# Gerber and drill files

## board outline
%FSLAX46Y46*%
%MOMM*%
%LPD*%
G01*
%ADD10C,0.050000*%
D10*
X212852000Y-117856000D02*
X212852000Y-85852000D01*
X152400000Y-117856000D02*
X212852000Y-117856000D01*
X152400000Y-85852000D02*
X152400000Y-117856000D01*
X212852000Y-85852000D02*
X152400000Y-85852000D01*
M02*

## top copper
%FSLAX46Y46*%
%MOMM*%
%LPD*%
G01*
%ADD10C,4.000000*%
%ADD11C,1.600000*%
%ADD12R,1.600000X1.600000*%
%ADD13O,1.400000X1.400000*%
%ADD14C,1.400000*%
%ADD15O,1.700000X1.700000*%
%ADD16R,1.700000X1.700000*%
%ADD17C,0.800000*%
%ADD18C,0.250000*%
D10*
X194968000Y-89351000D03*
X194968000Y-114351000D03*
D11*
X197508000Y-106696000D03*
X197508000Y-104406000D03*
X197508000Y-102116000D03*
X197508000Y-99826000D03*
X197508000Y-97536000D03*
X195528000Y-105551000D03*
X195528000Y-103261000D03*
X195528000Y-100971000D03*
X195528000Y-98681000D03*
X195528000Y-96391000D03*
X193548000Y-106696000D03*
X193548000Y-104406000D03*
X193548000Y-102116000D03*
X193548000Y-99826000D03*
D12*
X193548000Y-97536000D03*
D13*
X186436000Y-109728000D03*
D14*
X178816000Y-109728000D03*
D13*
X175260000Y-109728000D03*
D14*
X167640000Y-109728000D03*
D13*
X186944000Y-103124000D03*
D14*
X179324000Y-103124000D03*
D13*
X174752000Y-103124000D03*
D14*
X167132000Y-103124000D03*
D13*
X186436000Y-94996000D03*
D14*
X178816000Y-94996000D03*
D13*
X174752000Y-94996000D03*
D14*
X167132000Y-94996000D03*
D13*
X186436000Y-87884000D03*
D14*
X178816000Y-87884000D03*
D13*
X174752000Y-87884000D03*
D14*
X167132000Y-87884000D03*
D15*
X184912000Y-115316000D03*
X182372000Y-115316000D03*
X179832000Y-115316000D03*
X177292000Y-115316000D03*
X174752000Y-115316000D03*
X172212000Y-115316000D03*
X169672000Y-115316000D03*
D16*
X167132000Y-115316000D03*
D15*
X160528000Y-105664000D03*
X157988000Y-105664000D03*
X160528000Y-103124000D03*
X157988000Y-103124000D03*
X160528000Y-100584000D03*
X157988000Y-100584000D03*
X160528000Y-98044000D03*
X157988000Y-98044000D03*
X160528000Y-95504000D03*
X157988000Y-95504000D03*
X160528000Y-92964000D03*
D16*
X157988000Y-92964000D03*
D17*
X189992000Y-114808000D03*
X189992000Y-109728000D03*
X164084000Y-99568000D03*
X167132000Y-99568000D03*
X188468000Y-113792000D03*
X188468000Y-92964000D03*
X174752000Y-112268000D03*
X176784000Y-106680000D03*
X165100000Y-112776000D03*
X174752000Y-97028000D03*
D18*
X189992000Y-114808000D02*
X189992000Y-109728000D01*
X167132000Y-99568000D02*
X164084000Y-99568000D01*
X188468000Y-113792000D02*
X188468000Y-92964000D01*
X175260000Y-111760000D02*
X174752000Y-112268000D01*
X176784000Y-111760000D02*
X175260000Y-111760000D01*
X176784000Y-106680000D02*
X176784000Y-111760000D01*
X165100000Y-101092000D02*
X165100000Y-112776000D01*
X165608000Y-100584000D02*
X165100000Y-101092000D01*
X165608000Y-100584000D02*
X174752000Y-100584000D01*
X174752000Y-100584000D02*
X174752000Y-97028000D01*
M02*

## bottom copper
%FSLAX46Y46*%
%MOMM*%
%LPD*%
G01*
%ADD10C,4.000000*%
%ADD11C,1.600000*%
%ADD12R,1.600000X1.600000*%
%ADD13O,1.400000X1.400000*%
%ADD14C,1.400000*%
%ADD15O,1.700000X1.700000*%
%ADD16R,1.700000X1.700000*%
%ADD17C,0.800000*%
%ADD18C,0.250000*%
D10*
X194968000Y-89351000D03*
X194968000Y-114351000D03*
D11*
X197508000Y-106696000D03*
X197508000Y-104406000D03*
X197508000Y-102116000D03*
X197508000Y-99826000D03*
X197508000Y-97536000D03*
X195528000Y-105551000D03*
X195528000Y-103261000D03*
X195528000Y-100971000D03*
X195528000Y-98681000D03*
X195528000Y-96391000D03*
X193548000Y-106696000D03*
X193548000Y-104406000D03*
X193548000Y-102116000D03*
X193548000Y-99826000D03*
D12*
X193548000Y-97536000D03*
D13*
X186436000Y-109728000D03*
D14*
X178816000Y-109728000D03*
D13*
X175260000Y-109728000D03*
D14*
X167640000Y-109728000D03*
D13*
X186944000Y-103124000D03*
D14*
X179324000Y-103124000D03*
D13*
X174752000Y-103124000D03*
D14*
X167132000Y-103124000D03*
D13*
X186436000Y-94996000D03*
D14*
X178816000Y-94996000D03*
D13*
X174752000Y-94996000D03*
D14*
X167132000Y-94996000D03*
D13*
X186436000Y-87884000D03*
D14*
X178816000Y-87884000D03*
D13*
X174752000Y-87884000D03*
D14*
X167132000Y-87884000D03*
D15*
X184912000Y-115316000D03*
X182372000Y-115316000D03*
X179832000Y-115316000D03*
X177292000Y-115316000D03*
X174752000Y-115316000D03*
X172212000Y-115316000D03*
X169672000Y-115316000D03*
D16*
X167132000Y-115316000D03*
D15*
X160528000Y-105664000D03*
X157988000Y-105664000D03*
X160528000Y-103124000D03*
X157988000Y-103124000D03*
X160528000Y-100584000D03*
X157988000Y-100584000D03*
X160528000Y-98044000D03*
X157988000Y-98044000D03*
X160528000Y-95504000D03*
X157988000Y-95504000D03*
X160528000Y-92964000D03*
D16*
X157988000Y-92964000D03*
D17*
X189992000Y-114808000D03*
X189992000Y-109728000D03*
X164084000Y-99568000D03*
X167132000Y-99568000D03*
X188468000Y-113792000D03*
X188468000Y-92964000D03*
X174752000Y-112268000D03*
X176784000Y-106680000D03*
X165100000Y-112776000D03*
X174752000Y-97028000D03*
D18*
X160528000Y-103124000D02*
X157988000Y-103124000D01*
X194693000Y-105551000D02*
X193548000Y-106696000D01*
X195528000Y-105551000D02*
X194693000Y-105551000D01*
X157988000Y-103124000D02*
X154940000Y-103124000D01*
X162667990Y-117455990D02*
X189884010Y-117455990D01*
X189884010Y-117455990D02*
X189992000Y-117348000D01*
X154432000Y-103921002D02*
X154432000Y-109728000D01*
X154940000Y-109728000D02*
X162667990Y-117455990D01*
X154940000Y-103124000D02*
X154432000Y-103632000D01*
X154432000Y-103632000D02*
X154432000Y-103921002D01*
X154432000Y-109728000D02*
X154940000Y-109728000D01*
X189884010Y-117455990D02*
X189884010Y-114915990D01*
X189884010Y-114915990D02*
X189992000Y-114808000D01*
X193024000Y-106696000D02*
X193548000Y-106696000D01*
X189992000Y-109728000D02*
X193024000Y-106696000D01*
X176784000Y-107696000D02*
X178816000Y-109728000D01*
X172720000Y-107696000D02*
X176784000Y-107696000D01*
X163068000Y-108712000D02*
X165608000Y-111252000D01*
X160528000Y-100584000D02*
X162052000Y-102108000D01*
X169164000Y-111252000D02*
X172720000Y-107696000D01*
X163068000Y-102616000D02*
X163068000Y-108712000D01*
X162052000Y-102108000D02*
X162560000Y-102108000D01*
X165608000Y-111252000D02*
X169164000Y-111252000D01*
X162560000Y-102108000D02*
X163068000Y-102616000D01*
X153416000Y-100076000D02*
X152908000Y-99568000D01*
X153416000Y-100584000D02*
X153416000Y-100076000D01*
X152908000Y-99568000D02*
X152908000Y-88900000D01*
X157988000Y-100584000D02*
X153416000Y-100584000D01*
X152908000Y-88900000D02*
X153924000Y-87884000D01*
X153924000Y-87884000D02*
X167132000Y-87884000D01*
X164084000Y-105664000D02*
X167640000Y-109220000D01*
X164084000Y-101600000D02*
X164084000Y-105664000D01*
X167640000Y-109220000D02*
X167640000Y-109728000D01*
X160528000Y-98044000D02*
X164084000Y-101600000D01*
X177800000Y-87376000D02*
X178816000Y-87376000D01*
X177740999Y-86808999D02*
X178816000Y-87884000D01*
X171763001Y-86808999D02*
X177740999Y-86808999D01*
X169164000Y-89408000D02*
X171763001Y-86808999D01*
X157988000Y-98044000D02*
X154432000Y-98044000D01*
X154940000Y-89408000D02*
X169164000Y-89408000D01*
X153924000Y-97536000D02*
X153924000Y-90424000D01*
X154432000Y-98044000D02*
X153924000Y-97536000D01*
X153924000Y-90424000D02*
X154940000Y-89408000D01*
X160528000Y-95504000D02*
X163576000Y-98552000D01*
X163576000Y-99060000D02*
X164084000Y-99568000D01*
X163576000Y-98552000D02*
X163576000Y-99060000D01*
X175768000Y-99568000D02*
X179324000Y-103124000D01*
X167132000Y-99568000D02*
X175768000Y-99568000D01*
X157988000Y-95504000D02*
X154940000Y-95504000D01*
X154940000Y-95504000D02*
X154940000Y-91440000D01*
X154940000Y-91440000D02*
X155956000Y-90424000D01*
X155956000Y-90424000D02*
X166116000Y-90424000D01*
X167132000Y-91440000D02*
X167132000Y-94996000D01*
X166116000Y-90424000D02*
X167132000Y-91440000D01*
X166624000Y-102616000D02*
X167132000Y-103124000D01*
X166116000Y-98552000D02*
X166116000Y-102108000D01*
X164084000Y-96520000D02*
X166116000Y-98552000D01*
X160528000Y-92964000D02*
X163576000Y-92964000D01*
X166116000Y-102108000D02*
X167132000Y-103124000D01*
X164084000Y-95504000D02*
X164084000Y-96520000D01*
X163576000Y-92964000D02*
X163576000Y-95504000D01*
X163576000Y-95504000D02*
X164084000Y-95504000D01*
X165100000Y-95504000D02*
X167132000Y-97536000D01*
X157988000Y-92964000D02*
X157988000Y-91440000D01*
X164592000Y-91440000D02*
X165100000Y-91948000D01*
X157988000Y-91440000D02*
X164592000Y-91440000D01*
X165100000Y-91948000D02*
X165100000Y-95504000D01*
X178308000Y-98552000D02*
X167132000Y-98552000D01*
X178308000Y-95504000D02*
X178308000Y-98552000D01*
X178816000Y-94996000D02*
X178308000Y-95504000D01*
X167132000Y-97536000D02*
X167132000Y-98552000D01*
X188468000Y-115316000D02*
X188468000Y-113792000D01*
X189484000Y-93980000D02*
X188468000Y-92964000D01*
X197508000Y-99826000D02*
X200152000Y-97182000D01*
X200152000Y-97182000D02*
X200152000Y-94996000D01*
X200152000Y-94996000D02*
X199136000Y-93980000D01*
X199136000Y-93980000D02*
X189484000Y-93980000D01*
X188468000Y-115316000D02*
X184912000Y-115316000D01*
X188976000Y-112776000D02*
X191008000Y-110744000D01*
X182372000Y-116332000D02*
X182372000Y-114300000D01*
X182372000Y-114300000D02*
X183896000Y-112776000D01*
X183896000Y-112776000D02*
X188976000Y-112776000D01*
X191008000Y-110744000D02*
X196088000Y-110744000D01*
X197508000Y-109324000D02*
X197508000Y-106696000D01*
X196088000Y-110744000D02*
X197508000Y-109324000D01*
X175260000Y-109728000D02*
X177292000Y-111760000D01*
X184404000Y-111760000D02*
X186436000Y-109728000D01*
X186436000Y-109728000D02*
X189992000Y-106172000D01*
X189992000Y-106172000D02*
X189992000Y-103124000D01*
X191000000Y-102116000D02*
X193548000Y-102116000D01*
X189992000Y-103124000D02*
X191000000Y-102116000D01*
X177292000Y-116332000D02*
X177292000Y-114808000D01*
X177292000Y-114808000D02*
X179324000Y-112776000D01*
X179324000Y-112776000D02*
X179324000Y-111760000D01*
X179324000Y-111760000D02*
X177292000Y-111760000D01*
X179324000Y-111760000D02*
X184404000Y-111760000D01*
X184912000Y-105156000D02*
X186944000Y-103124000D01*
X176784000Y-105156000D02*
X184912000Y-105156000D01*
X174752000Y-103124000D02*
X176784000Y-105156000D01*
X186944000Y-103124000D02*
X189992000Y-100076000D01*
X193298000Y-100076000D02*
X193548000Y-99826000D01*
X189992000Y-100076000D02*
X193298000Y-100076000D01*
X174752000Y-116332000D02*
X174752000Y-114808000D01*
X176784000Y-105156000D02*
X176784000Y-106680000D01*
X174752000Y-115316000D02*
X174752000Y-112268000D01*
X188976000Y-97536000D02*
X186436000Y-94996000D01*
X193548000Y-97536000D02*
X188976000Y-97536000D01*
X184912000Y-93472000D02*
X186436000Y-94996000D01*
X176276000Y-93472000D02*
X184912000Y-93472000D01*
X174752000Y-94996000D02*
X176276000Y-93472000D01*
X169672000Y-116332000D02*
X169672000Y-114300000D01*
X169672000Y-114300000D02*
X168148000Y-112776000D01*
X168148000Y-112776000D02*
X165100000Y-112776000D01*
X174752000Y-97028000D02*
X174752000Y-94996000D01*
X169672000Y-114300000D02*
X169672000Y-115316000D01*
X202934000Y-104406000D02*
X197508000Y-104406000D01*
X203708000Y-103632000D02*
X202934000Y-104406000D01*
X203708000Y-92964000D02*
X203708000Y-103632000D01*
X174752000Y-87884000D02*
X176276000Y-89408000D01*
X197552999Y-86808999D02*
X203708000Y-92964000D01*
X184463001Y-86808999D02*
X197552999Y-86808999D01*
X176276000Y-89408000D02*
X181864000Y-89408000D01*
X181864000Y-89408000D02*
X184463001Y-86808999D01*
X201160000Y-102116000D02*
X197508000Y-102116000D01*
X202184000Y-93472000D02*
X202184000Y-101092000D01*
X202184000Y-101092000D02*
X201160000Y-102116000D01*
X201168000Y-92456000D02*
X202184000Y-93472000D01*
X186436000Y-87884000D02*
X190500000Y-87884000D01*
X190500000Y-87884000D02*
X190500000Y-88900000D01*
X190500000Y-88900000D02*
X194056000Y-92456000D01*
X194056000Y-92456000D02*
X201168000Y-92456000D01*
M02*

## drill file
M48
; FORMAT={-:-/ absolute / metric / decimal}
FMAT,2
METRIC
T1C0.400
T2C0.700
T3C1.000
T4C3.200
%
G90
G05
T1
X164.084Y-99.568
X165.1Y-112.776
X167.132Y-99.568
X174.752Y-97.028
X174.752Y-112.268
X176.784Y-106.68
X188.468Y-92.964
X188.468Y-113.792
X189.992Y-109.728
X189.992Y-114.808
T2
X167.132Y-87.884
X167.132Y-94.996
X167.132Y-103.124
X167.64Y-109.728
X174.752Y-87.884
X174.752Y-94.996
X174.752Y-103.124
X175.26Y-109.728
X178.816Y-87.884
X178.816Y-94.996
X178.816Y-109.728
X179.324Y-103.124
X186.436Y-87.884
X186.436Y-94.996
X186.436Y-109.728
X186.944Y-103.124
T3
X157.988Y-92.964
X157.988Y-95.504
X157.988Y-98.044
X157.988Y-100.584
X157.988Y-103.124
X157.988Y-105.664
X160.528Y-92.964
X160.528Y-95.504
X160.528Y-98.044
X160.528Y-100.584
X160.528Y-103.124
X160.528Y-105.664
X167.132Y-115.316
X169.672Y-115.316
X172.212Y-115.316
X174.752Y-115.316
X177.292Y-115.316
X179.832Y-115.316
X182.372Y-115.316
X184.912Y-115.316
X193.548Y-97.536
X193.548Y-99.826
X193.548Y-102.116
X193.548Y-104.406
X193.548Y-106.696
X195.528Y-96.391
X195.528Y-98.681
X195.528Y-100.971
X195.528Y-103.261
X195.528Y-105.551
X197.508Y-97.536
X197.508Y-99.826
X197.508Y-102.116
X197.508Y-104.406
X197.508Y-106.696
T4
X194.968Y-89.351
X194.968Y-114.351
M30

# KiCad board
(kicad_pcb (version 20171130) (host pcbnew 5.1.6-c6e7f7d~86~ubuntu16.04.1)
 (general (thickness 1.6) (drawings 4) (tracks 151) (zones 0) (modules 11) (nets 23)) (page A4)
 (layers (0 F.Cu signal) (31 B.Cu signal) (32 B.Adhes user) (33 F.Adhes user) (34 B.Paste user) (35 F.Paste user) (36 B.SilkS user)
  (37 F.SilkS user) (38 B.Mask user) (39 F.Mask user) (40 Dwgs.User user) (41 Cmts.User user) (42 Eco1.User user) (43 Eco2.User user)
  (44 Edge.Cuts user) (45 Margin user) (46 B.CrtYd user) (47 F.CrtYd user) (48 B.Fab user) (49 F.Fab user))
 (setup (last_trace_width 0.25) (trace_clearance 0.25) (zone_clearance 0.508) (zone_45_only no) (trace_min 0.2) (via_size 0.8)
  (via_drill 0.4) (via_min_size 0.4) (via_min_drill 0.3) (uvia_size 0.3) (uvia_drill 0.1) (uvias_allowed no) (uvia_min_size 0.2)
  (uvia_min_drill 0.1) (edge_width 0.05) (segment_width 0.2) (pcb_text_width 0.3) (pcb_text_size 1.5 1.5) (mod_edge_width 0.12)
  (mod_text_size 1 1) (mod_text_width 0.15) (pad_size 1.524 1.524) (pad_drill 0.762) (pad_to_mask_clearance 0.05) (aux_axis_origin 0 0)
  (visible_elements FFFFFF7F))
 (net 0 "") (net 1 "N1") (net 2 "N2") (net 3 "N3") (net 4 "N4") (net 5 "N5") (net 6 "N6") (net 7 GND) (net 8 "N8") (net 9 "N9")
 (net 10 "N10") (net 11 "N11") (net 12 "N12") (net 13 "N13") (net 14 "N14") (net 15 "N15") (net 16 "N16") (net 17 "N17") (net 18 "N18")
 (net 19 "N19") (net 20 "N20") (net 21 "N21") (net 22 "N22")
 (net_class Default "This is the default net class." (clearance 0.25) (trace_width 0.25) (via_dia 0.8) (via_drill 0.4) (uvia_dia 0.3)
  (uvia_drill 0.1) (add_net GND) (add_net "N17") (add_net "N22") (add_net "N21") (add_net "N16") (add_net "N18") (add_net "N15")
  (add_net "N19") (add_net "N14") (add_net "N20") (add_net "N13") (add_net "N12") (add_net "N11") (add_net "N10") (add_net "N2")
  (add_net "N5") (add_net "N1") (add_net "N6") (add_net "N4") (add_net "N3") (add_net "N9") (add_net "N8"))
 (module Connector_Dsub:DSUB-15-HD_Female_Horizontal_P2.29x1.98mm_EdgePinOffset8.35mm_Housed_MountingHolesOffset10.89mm (layer F.Cu)
  (at 193.548 97.536 90)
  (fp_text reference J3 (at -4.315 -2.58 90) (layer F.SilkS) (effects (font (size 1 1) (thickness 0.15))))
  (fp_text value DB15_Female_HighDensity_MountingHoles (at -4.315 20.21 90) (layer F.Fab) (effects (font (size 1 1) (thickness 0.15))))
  (pad 0 thru_hole circle (at 8.185 1.42 90) (size 4 4) (drill 3.2) (layers *.Cu *.Mask) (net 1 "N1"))
  (pad 0 thru_hole circle (at -16.815 1.42 90) (size 4 4) (drill 3.2) (layers *.Cu *.Mask) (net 1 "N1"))
  (pad 15 thru_hole circle (at -9.16 3.96 90) (size 1.6 1.6) (drill 1) (layers *.Cu *.Mask) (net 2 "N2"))
  (pad 14 thru_hole circle (at -6.87 3.96 90) (size 1.6 1.6) (drill 1) (layers *.Cu *.Mask) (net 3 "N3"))
  (pad 13 thru_hole circle (at -4.58 3.96 90) (size 1.6 1.6) (drill 1) (layers *.Cu *.Mask) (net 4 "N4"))
  (pad 12 thru_hole circle (at -2.29 3.96 90) (size 1.6 1.6) (drill 1) (layers *.Cu *.Mask) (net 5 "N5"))
  (pad 11 thru_hole circle (at 0 3.96 90) (size 1.6 1.6) (drill 1) (layers *.Cu *.Mask) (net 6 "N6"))
  (pad 10 thru_hole circle (at -8.015 1.98 90) (size 1.6 1.6) (drill 1) (layers *.Cu *.Mask) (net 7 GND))
  (pad 9 thru_hole circle (at -5.725 1.98 90) (size 1.6 1.6) (drill 1) (layers *.Cu *.Mask) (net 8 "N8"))
  (pad 8 thru_hole circle (at -3.435 1.98 90) (size 1.6 1.6) (drill 1) (layers *.Cu *.Mask) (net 7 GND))
  (pad 7 thru_hole circle (at -1.145 1.98 90) (size 1.6 1.6) (drill 1) (layers *.Cu *.Mask) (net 7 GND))
  (pad 6 thru_hole circle (at 1.145 1.98 90) (size 1.6 1.6) (drill 1) (layers *.Cu *.Mask) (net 7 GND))
  (pad 5 thru_hole circle (at -9.16 0 90) (size 1.6 1.6) (drill 1) (layers *.Cu *.Mask) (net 7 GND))
  (pad 4 thru_hole circle (at -6.87 0 90) (size 1.6 1.6) (drill 1) (layers *.Cu *.Mask) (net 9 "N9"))
  (pad 3 thru_hole circle (at -4.58 0 90) (size 1.6 1.6) (drill 1) (layers *.Cu *.Mask) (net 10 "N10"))
  (pad 2 thru_hole circle (at -2.29 0 90) (size 1.6 1.6) (drill 1) (layers *.Cu *.Mask) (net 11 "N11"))
  (pad 1 thru_hole rect (at 0 0 90) (size 1.6 1.6) (drill 1) (layers *.Cu *.Mask) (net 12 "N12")))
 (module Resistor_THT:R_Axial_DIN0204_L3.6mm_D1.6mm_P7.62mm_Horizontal (layer F.Cu) (at 178.816 109.728)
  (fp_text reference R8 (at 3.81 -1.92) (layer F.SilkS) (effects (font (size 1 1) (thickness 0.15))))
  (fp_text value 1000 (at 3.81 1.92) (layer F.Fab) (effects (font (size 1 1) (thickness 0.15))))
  (pad 2 thru_hole oval (at 7.62 0) (size 1.4 1.4) (drill 0.7) (layers *.Cu *.Mask) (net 10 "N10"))
  (pad 1 thru_hole circle (at 0 0) (size 1.4 1.4) (drill 0.7) (layers *.Cu *.Mask) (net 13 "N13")))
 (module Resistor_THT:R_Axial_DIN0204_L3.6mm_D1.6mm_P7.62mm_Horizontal (layer F.Cu) (at 167.64 109.728)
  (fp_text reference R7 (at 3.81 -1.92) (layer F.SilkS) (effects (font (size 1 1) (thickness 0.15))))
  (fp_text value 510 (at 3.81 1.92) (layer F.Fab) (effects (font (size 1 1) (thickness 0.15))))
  (pad 2 thru_hole oval (at 7.62 0) (size 1.4 1.4) (drill 0.7) (layers *.Cu *.Mask) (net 10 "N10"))
  (pad 1 thru_hole circle (at 0 0) (size 1.4 1.4) (drill 0.7) (layers *.Cu *.Mask) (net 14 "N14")))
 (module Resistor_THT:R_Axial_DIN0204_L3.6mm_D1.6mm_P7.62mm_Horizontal (layer F.Cu) (at 179.324 103.124)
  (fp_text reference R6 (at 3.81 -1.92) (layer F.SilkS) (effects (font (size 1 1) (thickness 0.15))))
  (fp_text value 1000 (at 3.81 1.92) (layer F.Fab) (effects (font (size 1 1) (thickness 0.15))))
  (pad 2 thru_hole oval (at 7.62 0) (size 1.4 1.4) (drill 0.7) (layers *.Cu *.Mask) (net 11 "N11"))
  (pad 1 thru_hole circle (at 0 0) (size 1.4 1.4) (drill 0.7) (layers *.Cu *.Mask) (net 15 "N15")))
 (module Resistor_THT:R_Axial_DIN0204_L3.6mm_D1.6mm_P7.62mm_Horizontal (layer F.Cu) (at 167.132 103.124)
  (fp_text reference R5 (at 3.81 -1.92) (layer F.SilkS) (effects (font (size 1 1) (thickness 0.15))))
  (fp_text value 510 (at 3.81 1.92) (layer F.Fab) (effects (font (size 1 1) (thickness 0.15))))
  (pad 2 thru_hole oval (at 7.62 0) (size 1.4 1.4) (drill 0.7) (layers *.Cu *.Mask) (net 11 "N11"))
  (pad 1 thru_hole circle (at 0 0) (size 1.4 1.4) (drill 0.7) (layers *.Cu *.Mask) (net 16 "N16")))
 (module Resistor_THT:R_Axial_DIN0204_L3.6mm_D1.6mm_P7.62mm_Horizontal (layer F.Cu) (at 178.816 94.996)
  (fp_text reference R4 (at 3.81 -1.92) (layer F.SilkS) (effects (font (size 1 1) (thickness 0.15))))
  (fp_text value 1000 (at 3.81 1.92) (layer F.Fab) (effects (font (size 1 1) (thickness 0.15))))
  (pad 2 thru_hole oval (at 7.62 0) (size 1.4 1.4) (drill 0.7) (layers *.Cu *.Mask) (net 12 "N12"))
  (pad 1 thru_hole circle (at 0 0) (size 1.4 1.4) (drill 0.7) (layers *.Cu *.Mask) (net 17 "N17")))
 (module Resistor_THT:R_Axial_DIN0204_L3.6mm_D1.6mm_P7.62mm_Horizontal (layer F.Cu) (at 167.132 94.996)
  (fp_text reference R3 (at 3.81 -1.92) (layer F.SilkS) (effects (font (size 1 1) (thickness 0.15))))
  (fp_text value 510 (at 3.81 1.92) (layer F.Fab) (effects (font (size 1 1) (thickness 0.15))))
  (pad 2 thru_hole oval (at 7.62 0) (size 1.4 1.4) (drill 0.7) (layers *.Cu *.Mask) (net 12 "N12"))
  (pad 1 thru_hole circle (at 0 0) (size 1.4 1.4) (drill 0.7) (layers *.Cu *.Mask) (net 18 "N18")))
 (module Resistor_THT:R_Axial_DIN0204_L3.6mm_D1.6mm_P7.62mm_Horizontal (layer F.Cu) (at 178.816 87.884)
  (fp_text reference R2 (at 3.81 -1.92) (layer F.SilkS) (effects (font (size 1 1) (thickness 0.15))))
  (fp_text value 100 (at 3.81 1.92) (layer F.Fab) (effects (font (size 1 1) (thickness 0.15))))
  (pad 2 thru_hole oval (at 7.62 0) (size 1.4 1.4) (drill 0.7) (layers *.Cu *.Mask) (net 4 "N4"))
  (pad 1 thru_hole circle (at 0 0) (size 1.4 1.4) (drill 0.7) (layers *.Cu *.Mask) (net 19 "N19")))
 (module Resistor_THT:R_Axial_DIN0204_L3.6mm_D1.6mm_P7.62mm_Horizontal (layer F.Cu) (at 167.132 87.884)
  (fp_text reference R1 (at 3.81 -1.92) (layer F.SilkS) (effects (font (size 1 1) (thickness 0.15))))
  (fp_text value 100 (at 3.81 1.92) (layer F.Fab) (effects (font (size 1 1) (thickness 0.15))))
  (pad 2 thru_hole oval (at 7.62 0) (size 1.4 1.4) (drill 0.7) (layers *.Cu *.Mask) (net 3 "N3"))
  (pad 1 thru_hole circle (at 0 0) (size 1.4 1.4) (drill 0.7) (layers *.Cu *.Mask) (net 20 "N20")))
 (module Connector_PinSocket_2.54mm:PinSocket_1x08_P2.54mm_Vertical (layer F.Cu) (at 167.132 115.316 90)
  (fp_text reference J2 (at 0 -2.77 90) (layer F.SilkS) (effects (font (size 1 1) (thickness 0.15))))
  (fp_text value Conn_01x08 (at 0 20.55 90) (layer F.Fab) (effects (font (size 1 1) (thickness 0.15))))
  (pad 8 thru_hole oval (at 0 17.78 90) (size 1.7 1.7) (drill 1) (layers *.Cu *.Mask) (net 5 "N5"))
  (pad 7 thru_hole oval (at 0 15.24 90) (size 1.7 1.7) (drill 1) (layers *.Cu *.Mask) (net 2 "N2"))
  (pad 6 thru_hole oval (at 0 12.7 90) (size 1.7 1.7) (drill 1) (layers *.Cu *.Mask) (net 10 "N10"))
  (pad 5 thru_hole oval (at 0 10.16 90) (size 1.7 1.7) (drill 1) (layers *.Cu *.Mask) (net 10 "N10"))
  (pad 4 thru_hole oval (at 0 7.62 90) (size 1.7 1.7) (drill 1) (layers *.Cu *.Mask) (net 11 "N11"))
  (pad 3 thru_hole oval (at 0 5.08 90) (size 1.7 1.7) (drill 1) (layers *.Cu *.Mask) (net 11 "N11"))
  (pad 2 thru_hole oval (at 0 2.54 90) (size 1.7 1.7) (drill 1) (layers *.Cu *.Mask) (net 12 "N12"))
  (pad 1 thru_hole rect (at 0 0 90) (size 1.7 1.7) (drill 1) (layers *.Cu *.Mask) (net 12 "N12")))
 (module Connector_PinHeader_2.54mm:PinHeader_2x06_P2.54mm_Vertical (layer F.Cu) (at 157.988 92.964)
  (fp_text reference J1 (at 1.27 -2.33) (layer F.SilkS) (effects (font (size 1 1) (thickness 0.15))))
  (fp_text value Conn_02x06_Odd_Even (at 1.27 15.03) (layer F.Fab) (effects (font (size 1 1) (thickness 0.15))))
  (pad 12 thru_hole oval (at 2.54 12.7) (size 1.7 1.7) (drill 1) (layers *.Cu *.Mask) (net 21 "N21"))
  (pad 11 thru_hole oval (at 0 12.7) (size 1.7 1.7) (drill 1) (layers *.Cu *.Mask) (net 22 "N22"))
  (pad 10 thru_hole oval (at 2.54 10.16) (size 1.7 1.7) (drill 1) (layers *.Cu *.Mask) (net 7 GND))
  (pad 9 thru_hole oval (at 0 10.16) (size 1.7 1.7) (drill 1) (layers *.Cu *.Mask) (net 7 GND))
  (pad 8 thru_hole oval (at 2.54 7.62) (size 1.7 1.7) (drill 1) (layers *.Cu *.Mask) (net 13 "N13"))
  (pad 7 thru_hole oval (at 0 7.62) (size 1.7 1.7) (drill 1) (layers *.Cu *.Mask) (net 20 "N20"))
  (pad 6 thru_hole oval (at 2.54 5.08) (size 1.7 1.7) (drill 1) (layers *.Cu *.Mask) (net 14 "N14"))
  (pad 5 thru_hole oval (at 0 5.08) (size 1.7 1.7) (drill 1) (layers *.Cu *.Mask) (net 19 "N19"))
  (pad 4 thru_hole oval (at 2.54 2.54) (size 1.7 1.7) (drill 1) (layers *.Cu *.Mask) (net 15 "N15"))
  (pad 3 thru_hole oval (at 0 2.54) (size 1.7 1.7) (drill 1) (layers *.Cu *.Mask) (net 18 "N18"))
  (pad 2 thru_hole oval (at 2.54 0) (size 1.7 1.7) (drill 1) (layers *.Cu *.Mask) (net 16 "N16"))
  (pad 1 thru_hole rect (at 0 0) (size 1.7 1.7) (drill 1) (layers *.Cu *.Mask) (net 17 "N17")))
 (gr_line (start 212.852 117.856) (end 212.852 85.852) (layer Edge.Cuts) (width 0.05))
 (gr_line (start 152.4 117.856) (end 212.852 117.856) (layer Edge.Cuts) (width 0.05))
 (gr_line (start 152.4 85.852) (end 152.4 117.856) (layer Edge.Cuts) (width 0.05))
 (gr_line (start 212.852 85.852) (end 152.4 85.852) (layer Edge.Cuts) (width 0.05))
 (segment (start 160.528 103.124) (end 157.988 103.124) (width 0.25) (layer B.Cu) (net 7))
 (segment (start 194.693 105.551) (end 193.548 106.696) (width 0.25) (layer B.Cu) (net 7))
 (segment (start 195.528 105.551) (end 194.693 105.551) (width 0.25) (layer B.Cu) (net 7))
 (segment (start 157.988 103.124) (end 154.94 103.124) (width 0.25) (layer B.Cu) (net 7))
 (segment (start 162.66799 117.45599) (end 189.88401 117.45599) (width 0.25) (layer B.Cu) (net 7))
 (segment (start 189.88401 117.45599) (end 189.992 117.348) (width 0.25) (layer B.Cu) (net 7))
 (segment (start 154.432 103.921002) (end 154.432 109.728) (width 0.25) (layer B.Cu) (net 7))
 (segment (start 154.94 109.728) (end 162.66799 117.45599) (width 0.25) (layer B.Cu) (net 7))
 (segment (start 154.94 103.124) (end 154.432 103.632) (width 0.25) (layer B.Cu) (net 7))
 (segment (start 154.432 103.632) (end 154.432 103.921002) (width 0.25) (layer B.Cu) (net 7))
 (segment (start 154.432 109.728) (end 154.94 109.728) (width 0.25) (layer B.Cu) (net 7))
 (segment (start 189.88401 117.45599) (end 189.88401 114.91599) (width 0.25) (layer B.Cu) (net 7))
 (via (at 189.992 114.808) (size 0.8) (drill 0.4) (layers F.Cu B.Cu) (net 7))
 (segment (start 189.88401 114.91599) (end 189.992 114.808) (width 0.25) (layer B.Cu) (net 7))
 (segment (start 189.992 114.808) (end 189.992 109.728) (width 0.25) (layer F.Cu) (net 7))
 (via (at 189.992 109.728) (size 0.8) (drill 0.4) (layers F.Cu B.Cu) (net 7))
 (segment (start 193.024 106.696) (end 193.548 106.696) (width 0.25) (layer B.Cu) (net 7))
 (segment (start 189.992 109.728) (end 193.024 106.696) (width 0.25) (layer B.Cu) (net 7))
 (segment (start 176.784 107.696) (end 178.816 109.728) (width 0.25) (layer B.Cu) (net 13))
 (segment (start 172.72 107.696) (end 176.784 107.696) (width 0.25) (layer B.Cu) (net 13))
 (segment (start 163.068 108.712) (end 165.608 111.252) (width 0.25) (layer B.Cu) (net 13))
 (segment (start 160.528 100.584) (end 162.052 102.108) (width 0.25) (layer B.Cu) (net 13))
 (segment (start 169.164 111.252) (end 172.72 107.696) (width 0.25) (layer B.Cu) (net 13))
 (segment (start 163.068 102.616) (end 163.068 108.712) (width 0.25) (layer B.Cu) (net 13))
 (segment (start 162.052 102.108) (end 162.56 102.108) (width 0.25) (layer B.Cu) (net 13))
 (segment (start 165.608 111.252) (end 169.164 111.252) (width 0.25) (layer B.Cu) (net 13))
 (segment (start 162.56 102.108) (end 163.068 102.616) (width 0.25) (layer B.Cu) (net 13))
 (segment (start 153.416 100.076) (end 152.908 99.568) (width 0.25) (layer B.Cu) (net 20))
 (segment (start 153.416 100.584) (end 153.416 100.076) (width 0.25) (layer B.Cu) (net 20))
 (segment (start 152.908 99.568) (end 152.908 88.9) (width 0.25) (layer B.Cu) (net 20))
 (segment (start 157.988 100.584) (end 153.416 100.584) (width 0.25) (layer B.Cu) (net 20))
 (segment (start 152.908 88.9) (end 153.924 87.884) (width 0.25) (layer B.Cu) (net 20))
 (segment (start 153.924 87.884) (end 167.132 87.884) (width 0.25) (layer B.Cu) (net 20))
 (segment (start 164.084 105.664) (end 167.64 109.22) (width 0.25) (layer B.Cu) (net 14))
 (segment (start 164.084 101.6) (end 164.084 105.664) (width 0.25) (layer B.Cu) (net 14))
 (segment (start 167.64 109.22) (end 167.64 109.728) (width 0.25) (layer B.Cu) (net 14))
 (segment (start 160.528 98.044) (end 164.084 101.6) (width 0.25) (layer B.Cu) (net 14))
 (segment (start 177.8 87.376) (end 178.816 87.376) (width 0.25) (layer B.Cu) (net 19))
 (segment (start 177.740999 86.808999) (end 178.816 87.884) (width 0.25) (layer B.Cu) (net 19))
 (segment (start 171.763001 86.808999) (end 177.740999 86.808999) (width 0.25) (layer B.Cu) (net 19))
 (segment (start 169.164 89.408) (end 171.763001 86.808999) (width 0.25) (layer B.Cu) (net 19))
 (segment (start 157.988 98.044) (end 154.432 98.044) (width 0.25) (layer B.Cu) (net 19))
 (segment (start 154.94 89.408) (end 169.164 89.408) (width 0.25) (layer B.Cu) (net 19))
 (segment (start 153.924 97.536) (end 153.924 90.424) (width 0.25) (layer B.Cu) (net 19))
 (segment (start 154.432 98.044) (end 153.924 97.536) (width 0.25) (layer B.Cu) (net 19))
 (segment (start 153.924 90.424) (end 154.94 89.408) (width 0.25) (layer B.Cu) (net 19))
 (segment (start 160.528 95.504) (end 163.576 98.552) (width 0.25) (layer B.Cu) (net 15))
 (via (at 164.084 99.568) (size 0.8) (drill 0.4) (layers F.Cu B.Cu) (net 15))
 (via (at 167.132 99.568) (size 0.8) (drill 0.4) (layers F.Cu B.Cu) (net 15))
 (segment (start 167.132 99.568) (end 164.084 99.568) (width 0.25) (layer F.Cu) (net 15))
 (segment (start 163.576 99.06) (end 164.084 99.568) (width 0.25) (layer B.Cu) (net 15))
 (segment (start 163.576 98.552) (end 163.576 99.06) (width 0.25) (layer B.Cu) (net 15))
 (segment (start 175.768 99.568) (end 179.324 103.124) (width 0.25) (layer B.Cu) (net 15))
 (segment (start 167.132 99.568) (end 175.768 99.568) (width 0.25) (layer B.Cu) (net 15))
 (segment (start 157.988 95.504) (end 154.94 95.504) (width 0.25) (layer B.Cu) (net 18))
 (segment (start 154.94 95.504) (end 154.94 91.44) (width 0.25) (layer B.Cu) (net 18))
 (segment (start 154.94 91.44) (end 155.956 90.424) (width 0.25) (layer B.Cu) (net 18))
 (segment (start 155.956 90.424) (end 166.116 90.424) (width 0.25) (layer B.Cu) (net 18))
 (segment (start 167.132 91.44) (end 167.132 94.996) (width 0.25) (layer B.Cu) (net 18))
 (segment (start 166.116 90.424) (end 167.132 91.44) (width 0.25) (layer B.Cu) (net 18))
 (segment (start 166.624 102.616) (end 167.132 103.124) (width 0.25) (layer B.Cu) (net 16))
 (segment (start 166.116 98.552) (end 166.116 102.108) (width 0.25) (layer B.Cu) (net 16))
 (segment (start 164.084 96.52) (end 166.116 98.552) (width 0.25) (layer B.Cu) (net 16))
 (segment (start 160.528 92.964) (end 163.576 92.964) (width 0.25) (layer B.Cu) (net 16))
 (segment (start 166.116 102.108) (end 167.132 103.124) (width 0.25) (layer B.Cu) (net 16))
 (segment (start 164.084 95.504) (end 164.084 96.52) (width 0.25) (layer B.Cu) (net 16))
 (segment (start 163.576 92.964) (end 163.576 95.504) (width 0.25) (layer B.Cu) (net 16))
 (segment (start 163.576 95.504) (end 164.084 95.504) (width 0.25) (layer B.Cu) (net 16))
 (segment (start 165.1 95.504) (end 167.132 97.536) (width 0.25) (layer B.Cu) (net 17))
 (segment (start 157.988 92.964) (end 157.988 91.44) (width 0.25) (layer B.Cu) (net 17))
 (segment (start 164.592 91.44) (end 165.1 91.948) (width 0.25) (layer B.Cu) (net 17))
 (segment (start 157.988 91.44) (end 164.592 91.44) (width 0.25) (layer B.Cu) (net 17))
 (segment (start 165.1 91.948) (end 165.1 95.504) (width 0.25) (layer B.Cu) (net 17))
 (segment (start 178.308 98.552) (end 167.132 98.552) (width 0.25) (layer B.Cu) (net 17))
 (segment (start 178.308 95.504) (end 178.308 98.552) (width 0.25) (layer B.Cu) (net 17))
 (segment (start 178.816 94.996) (end 178.308 95.504) (width 0.25) (layer B.Cu) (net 17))
 (segment (start 167.132 97.536) (end 167.132 98.552) (width 0.25) (layer B.Cu) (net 17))
 (via (at 188.468 113.792) (size 0.8) (drill 0.4) (layers F.Cu B.Cu) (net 5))
 (via (at 188.468 92.964) (size 0.8) (drill 0.4) (layers F.Cu B.Cu) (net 5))
 (segment (start 188.468 115.316) (end 188.468 113.792) (width 0.25) (layer B.Cu) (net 5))
 (segment (start 188.468 113.792) (end 188.468 92.964) (width 0.25) (layer F.Cu) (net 5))
 (segment (start 189.484 93.98) (end 188.468 92.964) (width 0.25) (layer B.Cu) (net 5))
 (segment (start 197.508 99.826) (end 200.152 97.182) (width 0.25) (layer B.Cu) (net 5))
 (segment (start 200.152 97.182) (end 200.152 94.996) (width 0.25) (layer B.Cu) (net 5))
 (segment (start 200.152 94.996) (end 199.136 93.98) (width 0.25) (layer B.Cu) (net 5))
 (segment (start 199.136 93.98) (end 189.484 93.98) (width 0.25) (layer B.Cu) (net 5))
 (segment (start 188.468 115.316) (end 184.912 115.316) (width 0.25) (layer B.Cu) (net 5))
 (segment (start 188.976 112.776) (end 191.008 110.744) (width 0.25) (layer B.Cu) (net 2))
 (segment (start 182.372 116.332) (end 182.372 114.3) (width 0.25) (layer B.Cu) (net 2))
 (segment (start 182.372 114.3) (end 183.896 112.776) (width 0.25) (layer B.Cu) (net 2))
 (segment (start 183.896 112.776) (end 188.976 112.776) (width 0.25) (layer B.Cu) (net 2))
 (segment (start 191.008 110.744) (end 196.088 110.744) (width 0.25) (layer B.Cu) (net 2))
 (segment (start 197.508 109.324) (end 197.508 106.696) (width 0.25) (layer B.Cu) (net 2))
 (segment (start 196.088 110.744) (end 197.508 109.324) (width 0.25) (layer B.Cu) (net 2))
 (segment (start 175.26 109.728) (end 177.292 111.76) (width 0.25) (layer B.Cu) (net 10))
 (segment (start 184.404 111.76) (end 186.436 109.728) (width 0.25) (layer B.Cu) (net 10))
 (segment (start 186.436 109.728) (end 189.992 106.172) (width 0.25) (layer B.Cu) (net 10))
 (segment (start 189.992 106.172) (end 189.992 103.124) (width 0.25) (layer B.Cu) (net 10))
 (segment (start 191 102.116) (end 193.548 102.116) (width 0.25) (layer B.Cu) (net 10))
 (segment (start 189.992 103.124) (end 191 102.116) (width 0.25) (layer B.Cu) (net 10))
 (segment (start 177.292 116.332) (end 177.292 114.808) (width 0.25) (layer B.Cu) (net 10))
 (segment (start 177.292 114.808) (end 179.324 112.776) (width 0.25) (layer B.Cu) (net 10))
 (segment (start 179.324 112.776) (end 179.324 111.76) (width 0.25) (layer B.Cu) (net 10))
 (segment (start 179.324 111.76) (end 177.292 111.76) (width 0.25) (layer B.Cu) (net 10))
 (segment (start 179.324 111.76) (end 184.404 111.76) (width 0.25) (layer B.Cu) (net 10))
 (segment (start 184.912 105.156) (end 186.944 103.124) (width 0.25) (layer B.Cu) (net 11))
 (segment (start 176.784 105.156) (end 184.912 105.156) (width 0.25) (layer B.Cu) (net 11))
 (segment (start 174.752 103.124) (end 176.784 105.156) (width 0.25) (layer B.Cu) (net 11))
 (segment (start 186.944 103.124) (end 189.992 100.076) (width 0.25) (layer B.Cu) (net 11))
 (segment (start 193.298 100.076) (end 193.548 99.826) (width 0.25) (layer B.Cu) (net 11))
 (segment (start 189.992 100.076) (end 193.298 100.076) (width 0.25) (layer B.Cu) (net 11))
 (segment (start 174.752 116.332) (end 174.752 114.808) (width 0.25) (layer B.Cu) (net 11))
 (via (at 174.752 112.268) (size 0.8) (drill 0.4) (layers F.Cu B.Cu) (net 11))
 (via (at 176.784 106.68) (size 0.8) (drill 0.4) (layers F.Cu B.Cu) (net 11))
 (segment (start 176.784 105.156) (end 176.784 106.68) (width 0.25) (layer B.Cu) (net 11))
 (segment (start 174.752 115.316) (end 174.752 112.268) (width 0.25) (layer B.Cu) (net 11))
 (segment (start 175.26 111.76) (end 174.752 112.268) (width 0.25) (layer F.Cu) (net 11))
 (segment (start 176.784 111.76) (end 175.26 111.76) (width 0.25) (layer F.Cu) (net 11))
 (segment (start 176.784 106.68) (end 176.784 111.76) (width 0.25) (layer F.Cu) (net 11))
 (segment (start 188.976 97.536) (end 186.436 94.996) (width 0.25) (layer B.Cu) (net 12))
 (segment (start 193.548 97.536) (end 188.976 97.536) (width 0.25) (layer B.Cu) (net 12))
 (segment (start 184.912 93.472) (end 186.436 94.996) (width 0.25) (layer B.Cu) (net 12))
 (segment (start 176.276 93.472) (end 184.912 93.472) (width 0.25) (layer B.Cu) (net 12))
 (segment (start 174.752 94.996) (end 176.276 93.472) (width 0.25) (layer B.Cu) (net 12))
 (segment (start 169.672 116.332) (end 169.672 114.3) (width 0.25) (layer B.Cu) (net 12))
 (segment (start 169.672 114.3) (end 168.148 112.776) (width 0.25) (layer B.Cu) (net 12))
 (via (at 165.1 112.776) (size 0.8) (drill 0.4) (layers F.Cu B.Cu) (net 12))
 (segment (start 168.148 112.776) (end 165.1 112.776) (width 0.25) (layer B.Cu) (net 12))
 (via (at 174.752 97.028) (size 0.8) (drill 0.4) (layers F.Cu B.Cu) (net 12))
 (segment (start 165.1 101.092) (end 165.1 112.776) (width 0.25) (layer F.Cu) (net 12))
 (segment (start 165.608 100.584) (end 165.1 101.092) (width 0.25) (layer F.Cu) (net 12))
 (segment (start 174.752 97.028) (end 174.752 94.996) (width 0.25) (layer B.Cu) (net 12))
 (segment (start 165.608 100.584) (end 174.752 100.584) (width 0.25) (layer F.Cu) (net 12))
 (segment (start 174.752 100.584) (end 174.752 97.028) (width 0.25) (layer F.Cu) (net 12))
 (segment (start 169.672 114.3) (end 169.672 115.316) (width 0.25) (layer B.Cu) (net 12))
 (segment (start 202.934 104.406) (end 197.508 104.406) (width 0.25) (layer B.Cu) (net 3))
 (segment (start 203.708 103.632) (end 202.934 104.406) (width 0.25) (layer B.Cu) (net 3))
 (segment (start 203.708 92.964) (end 203.708 103.632) (width 0.25) (layer B.Cu) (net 3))
 (segment (start 174.752 87.884) (end 176.276 89.408) (width 0.25) (layer B.Cu) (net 3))
 (segment (start 197.552999 86.808999) (end 203.708 92.964) (width 0.25) (layer B.Cu) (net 3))
 (segment (start 184.463001 86.808999) (end 197.552999 86.808999) (width 0.25) (layer B.Cu) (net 3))
 (segment (start 176.276 89.408) (end 181.864 89.408) (width 0.25) (layer B.Cu) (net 3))
 (segment (start 181.864 89.408) (end 184.463001 86.808999) (width 0.25) (layer B.Cu) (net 3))
 (segment (start 201.16 102.116) (end 197.508 102.116) (width 0.25) (layer B.Cu) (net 4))
 (segment (start 202.184 93.472) (end 202.184 101.092) (width 0.25) (layer B.Cu) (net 4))
 (segment (start 202.184 101.092) (end 201.16 102.116) (width 0.25) (layer B.Cu) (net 4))
 (segment (start 201.168 92.456) (end 202.184 93.472) (width 0.25) (layer B.Cu) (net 4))
 (segment (start 186.436 87.884) (end 190.5 87.884) (width 0.25) (layer B.Cu) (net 4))
 (segment (start 190.5 87.884) (end 190.5 88.9) (width 0.25) (layer B.Cu) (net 4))
 (segment (start 190.5 88.9) (end 194.056 92.456) (width 0.25) (layer B.Cu) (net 4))
 (segment (start 194.056 92.456) (end 201.168 92.456) (width 0.25) (layer B.Cu) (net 4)))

